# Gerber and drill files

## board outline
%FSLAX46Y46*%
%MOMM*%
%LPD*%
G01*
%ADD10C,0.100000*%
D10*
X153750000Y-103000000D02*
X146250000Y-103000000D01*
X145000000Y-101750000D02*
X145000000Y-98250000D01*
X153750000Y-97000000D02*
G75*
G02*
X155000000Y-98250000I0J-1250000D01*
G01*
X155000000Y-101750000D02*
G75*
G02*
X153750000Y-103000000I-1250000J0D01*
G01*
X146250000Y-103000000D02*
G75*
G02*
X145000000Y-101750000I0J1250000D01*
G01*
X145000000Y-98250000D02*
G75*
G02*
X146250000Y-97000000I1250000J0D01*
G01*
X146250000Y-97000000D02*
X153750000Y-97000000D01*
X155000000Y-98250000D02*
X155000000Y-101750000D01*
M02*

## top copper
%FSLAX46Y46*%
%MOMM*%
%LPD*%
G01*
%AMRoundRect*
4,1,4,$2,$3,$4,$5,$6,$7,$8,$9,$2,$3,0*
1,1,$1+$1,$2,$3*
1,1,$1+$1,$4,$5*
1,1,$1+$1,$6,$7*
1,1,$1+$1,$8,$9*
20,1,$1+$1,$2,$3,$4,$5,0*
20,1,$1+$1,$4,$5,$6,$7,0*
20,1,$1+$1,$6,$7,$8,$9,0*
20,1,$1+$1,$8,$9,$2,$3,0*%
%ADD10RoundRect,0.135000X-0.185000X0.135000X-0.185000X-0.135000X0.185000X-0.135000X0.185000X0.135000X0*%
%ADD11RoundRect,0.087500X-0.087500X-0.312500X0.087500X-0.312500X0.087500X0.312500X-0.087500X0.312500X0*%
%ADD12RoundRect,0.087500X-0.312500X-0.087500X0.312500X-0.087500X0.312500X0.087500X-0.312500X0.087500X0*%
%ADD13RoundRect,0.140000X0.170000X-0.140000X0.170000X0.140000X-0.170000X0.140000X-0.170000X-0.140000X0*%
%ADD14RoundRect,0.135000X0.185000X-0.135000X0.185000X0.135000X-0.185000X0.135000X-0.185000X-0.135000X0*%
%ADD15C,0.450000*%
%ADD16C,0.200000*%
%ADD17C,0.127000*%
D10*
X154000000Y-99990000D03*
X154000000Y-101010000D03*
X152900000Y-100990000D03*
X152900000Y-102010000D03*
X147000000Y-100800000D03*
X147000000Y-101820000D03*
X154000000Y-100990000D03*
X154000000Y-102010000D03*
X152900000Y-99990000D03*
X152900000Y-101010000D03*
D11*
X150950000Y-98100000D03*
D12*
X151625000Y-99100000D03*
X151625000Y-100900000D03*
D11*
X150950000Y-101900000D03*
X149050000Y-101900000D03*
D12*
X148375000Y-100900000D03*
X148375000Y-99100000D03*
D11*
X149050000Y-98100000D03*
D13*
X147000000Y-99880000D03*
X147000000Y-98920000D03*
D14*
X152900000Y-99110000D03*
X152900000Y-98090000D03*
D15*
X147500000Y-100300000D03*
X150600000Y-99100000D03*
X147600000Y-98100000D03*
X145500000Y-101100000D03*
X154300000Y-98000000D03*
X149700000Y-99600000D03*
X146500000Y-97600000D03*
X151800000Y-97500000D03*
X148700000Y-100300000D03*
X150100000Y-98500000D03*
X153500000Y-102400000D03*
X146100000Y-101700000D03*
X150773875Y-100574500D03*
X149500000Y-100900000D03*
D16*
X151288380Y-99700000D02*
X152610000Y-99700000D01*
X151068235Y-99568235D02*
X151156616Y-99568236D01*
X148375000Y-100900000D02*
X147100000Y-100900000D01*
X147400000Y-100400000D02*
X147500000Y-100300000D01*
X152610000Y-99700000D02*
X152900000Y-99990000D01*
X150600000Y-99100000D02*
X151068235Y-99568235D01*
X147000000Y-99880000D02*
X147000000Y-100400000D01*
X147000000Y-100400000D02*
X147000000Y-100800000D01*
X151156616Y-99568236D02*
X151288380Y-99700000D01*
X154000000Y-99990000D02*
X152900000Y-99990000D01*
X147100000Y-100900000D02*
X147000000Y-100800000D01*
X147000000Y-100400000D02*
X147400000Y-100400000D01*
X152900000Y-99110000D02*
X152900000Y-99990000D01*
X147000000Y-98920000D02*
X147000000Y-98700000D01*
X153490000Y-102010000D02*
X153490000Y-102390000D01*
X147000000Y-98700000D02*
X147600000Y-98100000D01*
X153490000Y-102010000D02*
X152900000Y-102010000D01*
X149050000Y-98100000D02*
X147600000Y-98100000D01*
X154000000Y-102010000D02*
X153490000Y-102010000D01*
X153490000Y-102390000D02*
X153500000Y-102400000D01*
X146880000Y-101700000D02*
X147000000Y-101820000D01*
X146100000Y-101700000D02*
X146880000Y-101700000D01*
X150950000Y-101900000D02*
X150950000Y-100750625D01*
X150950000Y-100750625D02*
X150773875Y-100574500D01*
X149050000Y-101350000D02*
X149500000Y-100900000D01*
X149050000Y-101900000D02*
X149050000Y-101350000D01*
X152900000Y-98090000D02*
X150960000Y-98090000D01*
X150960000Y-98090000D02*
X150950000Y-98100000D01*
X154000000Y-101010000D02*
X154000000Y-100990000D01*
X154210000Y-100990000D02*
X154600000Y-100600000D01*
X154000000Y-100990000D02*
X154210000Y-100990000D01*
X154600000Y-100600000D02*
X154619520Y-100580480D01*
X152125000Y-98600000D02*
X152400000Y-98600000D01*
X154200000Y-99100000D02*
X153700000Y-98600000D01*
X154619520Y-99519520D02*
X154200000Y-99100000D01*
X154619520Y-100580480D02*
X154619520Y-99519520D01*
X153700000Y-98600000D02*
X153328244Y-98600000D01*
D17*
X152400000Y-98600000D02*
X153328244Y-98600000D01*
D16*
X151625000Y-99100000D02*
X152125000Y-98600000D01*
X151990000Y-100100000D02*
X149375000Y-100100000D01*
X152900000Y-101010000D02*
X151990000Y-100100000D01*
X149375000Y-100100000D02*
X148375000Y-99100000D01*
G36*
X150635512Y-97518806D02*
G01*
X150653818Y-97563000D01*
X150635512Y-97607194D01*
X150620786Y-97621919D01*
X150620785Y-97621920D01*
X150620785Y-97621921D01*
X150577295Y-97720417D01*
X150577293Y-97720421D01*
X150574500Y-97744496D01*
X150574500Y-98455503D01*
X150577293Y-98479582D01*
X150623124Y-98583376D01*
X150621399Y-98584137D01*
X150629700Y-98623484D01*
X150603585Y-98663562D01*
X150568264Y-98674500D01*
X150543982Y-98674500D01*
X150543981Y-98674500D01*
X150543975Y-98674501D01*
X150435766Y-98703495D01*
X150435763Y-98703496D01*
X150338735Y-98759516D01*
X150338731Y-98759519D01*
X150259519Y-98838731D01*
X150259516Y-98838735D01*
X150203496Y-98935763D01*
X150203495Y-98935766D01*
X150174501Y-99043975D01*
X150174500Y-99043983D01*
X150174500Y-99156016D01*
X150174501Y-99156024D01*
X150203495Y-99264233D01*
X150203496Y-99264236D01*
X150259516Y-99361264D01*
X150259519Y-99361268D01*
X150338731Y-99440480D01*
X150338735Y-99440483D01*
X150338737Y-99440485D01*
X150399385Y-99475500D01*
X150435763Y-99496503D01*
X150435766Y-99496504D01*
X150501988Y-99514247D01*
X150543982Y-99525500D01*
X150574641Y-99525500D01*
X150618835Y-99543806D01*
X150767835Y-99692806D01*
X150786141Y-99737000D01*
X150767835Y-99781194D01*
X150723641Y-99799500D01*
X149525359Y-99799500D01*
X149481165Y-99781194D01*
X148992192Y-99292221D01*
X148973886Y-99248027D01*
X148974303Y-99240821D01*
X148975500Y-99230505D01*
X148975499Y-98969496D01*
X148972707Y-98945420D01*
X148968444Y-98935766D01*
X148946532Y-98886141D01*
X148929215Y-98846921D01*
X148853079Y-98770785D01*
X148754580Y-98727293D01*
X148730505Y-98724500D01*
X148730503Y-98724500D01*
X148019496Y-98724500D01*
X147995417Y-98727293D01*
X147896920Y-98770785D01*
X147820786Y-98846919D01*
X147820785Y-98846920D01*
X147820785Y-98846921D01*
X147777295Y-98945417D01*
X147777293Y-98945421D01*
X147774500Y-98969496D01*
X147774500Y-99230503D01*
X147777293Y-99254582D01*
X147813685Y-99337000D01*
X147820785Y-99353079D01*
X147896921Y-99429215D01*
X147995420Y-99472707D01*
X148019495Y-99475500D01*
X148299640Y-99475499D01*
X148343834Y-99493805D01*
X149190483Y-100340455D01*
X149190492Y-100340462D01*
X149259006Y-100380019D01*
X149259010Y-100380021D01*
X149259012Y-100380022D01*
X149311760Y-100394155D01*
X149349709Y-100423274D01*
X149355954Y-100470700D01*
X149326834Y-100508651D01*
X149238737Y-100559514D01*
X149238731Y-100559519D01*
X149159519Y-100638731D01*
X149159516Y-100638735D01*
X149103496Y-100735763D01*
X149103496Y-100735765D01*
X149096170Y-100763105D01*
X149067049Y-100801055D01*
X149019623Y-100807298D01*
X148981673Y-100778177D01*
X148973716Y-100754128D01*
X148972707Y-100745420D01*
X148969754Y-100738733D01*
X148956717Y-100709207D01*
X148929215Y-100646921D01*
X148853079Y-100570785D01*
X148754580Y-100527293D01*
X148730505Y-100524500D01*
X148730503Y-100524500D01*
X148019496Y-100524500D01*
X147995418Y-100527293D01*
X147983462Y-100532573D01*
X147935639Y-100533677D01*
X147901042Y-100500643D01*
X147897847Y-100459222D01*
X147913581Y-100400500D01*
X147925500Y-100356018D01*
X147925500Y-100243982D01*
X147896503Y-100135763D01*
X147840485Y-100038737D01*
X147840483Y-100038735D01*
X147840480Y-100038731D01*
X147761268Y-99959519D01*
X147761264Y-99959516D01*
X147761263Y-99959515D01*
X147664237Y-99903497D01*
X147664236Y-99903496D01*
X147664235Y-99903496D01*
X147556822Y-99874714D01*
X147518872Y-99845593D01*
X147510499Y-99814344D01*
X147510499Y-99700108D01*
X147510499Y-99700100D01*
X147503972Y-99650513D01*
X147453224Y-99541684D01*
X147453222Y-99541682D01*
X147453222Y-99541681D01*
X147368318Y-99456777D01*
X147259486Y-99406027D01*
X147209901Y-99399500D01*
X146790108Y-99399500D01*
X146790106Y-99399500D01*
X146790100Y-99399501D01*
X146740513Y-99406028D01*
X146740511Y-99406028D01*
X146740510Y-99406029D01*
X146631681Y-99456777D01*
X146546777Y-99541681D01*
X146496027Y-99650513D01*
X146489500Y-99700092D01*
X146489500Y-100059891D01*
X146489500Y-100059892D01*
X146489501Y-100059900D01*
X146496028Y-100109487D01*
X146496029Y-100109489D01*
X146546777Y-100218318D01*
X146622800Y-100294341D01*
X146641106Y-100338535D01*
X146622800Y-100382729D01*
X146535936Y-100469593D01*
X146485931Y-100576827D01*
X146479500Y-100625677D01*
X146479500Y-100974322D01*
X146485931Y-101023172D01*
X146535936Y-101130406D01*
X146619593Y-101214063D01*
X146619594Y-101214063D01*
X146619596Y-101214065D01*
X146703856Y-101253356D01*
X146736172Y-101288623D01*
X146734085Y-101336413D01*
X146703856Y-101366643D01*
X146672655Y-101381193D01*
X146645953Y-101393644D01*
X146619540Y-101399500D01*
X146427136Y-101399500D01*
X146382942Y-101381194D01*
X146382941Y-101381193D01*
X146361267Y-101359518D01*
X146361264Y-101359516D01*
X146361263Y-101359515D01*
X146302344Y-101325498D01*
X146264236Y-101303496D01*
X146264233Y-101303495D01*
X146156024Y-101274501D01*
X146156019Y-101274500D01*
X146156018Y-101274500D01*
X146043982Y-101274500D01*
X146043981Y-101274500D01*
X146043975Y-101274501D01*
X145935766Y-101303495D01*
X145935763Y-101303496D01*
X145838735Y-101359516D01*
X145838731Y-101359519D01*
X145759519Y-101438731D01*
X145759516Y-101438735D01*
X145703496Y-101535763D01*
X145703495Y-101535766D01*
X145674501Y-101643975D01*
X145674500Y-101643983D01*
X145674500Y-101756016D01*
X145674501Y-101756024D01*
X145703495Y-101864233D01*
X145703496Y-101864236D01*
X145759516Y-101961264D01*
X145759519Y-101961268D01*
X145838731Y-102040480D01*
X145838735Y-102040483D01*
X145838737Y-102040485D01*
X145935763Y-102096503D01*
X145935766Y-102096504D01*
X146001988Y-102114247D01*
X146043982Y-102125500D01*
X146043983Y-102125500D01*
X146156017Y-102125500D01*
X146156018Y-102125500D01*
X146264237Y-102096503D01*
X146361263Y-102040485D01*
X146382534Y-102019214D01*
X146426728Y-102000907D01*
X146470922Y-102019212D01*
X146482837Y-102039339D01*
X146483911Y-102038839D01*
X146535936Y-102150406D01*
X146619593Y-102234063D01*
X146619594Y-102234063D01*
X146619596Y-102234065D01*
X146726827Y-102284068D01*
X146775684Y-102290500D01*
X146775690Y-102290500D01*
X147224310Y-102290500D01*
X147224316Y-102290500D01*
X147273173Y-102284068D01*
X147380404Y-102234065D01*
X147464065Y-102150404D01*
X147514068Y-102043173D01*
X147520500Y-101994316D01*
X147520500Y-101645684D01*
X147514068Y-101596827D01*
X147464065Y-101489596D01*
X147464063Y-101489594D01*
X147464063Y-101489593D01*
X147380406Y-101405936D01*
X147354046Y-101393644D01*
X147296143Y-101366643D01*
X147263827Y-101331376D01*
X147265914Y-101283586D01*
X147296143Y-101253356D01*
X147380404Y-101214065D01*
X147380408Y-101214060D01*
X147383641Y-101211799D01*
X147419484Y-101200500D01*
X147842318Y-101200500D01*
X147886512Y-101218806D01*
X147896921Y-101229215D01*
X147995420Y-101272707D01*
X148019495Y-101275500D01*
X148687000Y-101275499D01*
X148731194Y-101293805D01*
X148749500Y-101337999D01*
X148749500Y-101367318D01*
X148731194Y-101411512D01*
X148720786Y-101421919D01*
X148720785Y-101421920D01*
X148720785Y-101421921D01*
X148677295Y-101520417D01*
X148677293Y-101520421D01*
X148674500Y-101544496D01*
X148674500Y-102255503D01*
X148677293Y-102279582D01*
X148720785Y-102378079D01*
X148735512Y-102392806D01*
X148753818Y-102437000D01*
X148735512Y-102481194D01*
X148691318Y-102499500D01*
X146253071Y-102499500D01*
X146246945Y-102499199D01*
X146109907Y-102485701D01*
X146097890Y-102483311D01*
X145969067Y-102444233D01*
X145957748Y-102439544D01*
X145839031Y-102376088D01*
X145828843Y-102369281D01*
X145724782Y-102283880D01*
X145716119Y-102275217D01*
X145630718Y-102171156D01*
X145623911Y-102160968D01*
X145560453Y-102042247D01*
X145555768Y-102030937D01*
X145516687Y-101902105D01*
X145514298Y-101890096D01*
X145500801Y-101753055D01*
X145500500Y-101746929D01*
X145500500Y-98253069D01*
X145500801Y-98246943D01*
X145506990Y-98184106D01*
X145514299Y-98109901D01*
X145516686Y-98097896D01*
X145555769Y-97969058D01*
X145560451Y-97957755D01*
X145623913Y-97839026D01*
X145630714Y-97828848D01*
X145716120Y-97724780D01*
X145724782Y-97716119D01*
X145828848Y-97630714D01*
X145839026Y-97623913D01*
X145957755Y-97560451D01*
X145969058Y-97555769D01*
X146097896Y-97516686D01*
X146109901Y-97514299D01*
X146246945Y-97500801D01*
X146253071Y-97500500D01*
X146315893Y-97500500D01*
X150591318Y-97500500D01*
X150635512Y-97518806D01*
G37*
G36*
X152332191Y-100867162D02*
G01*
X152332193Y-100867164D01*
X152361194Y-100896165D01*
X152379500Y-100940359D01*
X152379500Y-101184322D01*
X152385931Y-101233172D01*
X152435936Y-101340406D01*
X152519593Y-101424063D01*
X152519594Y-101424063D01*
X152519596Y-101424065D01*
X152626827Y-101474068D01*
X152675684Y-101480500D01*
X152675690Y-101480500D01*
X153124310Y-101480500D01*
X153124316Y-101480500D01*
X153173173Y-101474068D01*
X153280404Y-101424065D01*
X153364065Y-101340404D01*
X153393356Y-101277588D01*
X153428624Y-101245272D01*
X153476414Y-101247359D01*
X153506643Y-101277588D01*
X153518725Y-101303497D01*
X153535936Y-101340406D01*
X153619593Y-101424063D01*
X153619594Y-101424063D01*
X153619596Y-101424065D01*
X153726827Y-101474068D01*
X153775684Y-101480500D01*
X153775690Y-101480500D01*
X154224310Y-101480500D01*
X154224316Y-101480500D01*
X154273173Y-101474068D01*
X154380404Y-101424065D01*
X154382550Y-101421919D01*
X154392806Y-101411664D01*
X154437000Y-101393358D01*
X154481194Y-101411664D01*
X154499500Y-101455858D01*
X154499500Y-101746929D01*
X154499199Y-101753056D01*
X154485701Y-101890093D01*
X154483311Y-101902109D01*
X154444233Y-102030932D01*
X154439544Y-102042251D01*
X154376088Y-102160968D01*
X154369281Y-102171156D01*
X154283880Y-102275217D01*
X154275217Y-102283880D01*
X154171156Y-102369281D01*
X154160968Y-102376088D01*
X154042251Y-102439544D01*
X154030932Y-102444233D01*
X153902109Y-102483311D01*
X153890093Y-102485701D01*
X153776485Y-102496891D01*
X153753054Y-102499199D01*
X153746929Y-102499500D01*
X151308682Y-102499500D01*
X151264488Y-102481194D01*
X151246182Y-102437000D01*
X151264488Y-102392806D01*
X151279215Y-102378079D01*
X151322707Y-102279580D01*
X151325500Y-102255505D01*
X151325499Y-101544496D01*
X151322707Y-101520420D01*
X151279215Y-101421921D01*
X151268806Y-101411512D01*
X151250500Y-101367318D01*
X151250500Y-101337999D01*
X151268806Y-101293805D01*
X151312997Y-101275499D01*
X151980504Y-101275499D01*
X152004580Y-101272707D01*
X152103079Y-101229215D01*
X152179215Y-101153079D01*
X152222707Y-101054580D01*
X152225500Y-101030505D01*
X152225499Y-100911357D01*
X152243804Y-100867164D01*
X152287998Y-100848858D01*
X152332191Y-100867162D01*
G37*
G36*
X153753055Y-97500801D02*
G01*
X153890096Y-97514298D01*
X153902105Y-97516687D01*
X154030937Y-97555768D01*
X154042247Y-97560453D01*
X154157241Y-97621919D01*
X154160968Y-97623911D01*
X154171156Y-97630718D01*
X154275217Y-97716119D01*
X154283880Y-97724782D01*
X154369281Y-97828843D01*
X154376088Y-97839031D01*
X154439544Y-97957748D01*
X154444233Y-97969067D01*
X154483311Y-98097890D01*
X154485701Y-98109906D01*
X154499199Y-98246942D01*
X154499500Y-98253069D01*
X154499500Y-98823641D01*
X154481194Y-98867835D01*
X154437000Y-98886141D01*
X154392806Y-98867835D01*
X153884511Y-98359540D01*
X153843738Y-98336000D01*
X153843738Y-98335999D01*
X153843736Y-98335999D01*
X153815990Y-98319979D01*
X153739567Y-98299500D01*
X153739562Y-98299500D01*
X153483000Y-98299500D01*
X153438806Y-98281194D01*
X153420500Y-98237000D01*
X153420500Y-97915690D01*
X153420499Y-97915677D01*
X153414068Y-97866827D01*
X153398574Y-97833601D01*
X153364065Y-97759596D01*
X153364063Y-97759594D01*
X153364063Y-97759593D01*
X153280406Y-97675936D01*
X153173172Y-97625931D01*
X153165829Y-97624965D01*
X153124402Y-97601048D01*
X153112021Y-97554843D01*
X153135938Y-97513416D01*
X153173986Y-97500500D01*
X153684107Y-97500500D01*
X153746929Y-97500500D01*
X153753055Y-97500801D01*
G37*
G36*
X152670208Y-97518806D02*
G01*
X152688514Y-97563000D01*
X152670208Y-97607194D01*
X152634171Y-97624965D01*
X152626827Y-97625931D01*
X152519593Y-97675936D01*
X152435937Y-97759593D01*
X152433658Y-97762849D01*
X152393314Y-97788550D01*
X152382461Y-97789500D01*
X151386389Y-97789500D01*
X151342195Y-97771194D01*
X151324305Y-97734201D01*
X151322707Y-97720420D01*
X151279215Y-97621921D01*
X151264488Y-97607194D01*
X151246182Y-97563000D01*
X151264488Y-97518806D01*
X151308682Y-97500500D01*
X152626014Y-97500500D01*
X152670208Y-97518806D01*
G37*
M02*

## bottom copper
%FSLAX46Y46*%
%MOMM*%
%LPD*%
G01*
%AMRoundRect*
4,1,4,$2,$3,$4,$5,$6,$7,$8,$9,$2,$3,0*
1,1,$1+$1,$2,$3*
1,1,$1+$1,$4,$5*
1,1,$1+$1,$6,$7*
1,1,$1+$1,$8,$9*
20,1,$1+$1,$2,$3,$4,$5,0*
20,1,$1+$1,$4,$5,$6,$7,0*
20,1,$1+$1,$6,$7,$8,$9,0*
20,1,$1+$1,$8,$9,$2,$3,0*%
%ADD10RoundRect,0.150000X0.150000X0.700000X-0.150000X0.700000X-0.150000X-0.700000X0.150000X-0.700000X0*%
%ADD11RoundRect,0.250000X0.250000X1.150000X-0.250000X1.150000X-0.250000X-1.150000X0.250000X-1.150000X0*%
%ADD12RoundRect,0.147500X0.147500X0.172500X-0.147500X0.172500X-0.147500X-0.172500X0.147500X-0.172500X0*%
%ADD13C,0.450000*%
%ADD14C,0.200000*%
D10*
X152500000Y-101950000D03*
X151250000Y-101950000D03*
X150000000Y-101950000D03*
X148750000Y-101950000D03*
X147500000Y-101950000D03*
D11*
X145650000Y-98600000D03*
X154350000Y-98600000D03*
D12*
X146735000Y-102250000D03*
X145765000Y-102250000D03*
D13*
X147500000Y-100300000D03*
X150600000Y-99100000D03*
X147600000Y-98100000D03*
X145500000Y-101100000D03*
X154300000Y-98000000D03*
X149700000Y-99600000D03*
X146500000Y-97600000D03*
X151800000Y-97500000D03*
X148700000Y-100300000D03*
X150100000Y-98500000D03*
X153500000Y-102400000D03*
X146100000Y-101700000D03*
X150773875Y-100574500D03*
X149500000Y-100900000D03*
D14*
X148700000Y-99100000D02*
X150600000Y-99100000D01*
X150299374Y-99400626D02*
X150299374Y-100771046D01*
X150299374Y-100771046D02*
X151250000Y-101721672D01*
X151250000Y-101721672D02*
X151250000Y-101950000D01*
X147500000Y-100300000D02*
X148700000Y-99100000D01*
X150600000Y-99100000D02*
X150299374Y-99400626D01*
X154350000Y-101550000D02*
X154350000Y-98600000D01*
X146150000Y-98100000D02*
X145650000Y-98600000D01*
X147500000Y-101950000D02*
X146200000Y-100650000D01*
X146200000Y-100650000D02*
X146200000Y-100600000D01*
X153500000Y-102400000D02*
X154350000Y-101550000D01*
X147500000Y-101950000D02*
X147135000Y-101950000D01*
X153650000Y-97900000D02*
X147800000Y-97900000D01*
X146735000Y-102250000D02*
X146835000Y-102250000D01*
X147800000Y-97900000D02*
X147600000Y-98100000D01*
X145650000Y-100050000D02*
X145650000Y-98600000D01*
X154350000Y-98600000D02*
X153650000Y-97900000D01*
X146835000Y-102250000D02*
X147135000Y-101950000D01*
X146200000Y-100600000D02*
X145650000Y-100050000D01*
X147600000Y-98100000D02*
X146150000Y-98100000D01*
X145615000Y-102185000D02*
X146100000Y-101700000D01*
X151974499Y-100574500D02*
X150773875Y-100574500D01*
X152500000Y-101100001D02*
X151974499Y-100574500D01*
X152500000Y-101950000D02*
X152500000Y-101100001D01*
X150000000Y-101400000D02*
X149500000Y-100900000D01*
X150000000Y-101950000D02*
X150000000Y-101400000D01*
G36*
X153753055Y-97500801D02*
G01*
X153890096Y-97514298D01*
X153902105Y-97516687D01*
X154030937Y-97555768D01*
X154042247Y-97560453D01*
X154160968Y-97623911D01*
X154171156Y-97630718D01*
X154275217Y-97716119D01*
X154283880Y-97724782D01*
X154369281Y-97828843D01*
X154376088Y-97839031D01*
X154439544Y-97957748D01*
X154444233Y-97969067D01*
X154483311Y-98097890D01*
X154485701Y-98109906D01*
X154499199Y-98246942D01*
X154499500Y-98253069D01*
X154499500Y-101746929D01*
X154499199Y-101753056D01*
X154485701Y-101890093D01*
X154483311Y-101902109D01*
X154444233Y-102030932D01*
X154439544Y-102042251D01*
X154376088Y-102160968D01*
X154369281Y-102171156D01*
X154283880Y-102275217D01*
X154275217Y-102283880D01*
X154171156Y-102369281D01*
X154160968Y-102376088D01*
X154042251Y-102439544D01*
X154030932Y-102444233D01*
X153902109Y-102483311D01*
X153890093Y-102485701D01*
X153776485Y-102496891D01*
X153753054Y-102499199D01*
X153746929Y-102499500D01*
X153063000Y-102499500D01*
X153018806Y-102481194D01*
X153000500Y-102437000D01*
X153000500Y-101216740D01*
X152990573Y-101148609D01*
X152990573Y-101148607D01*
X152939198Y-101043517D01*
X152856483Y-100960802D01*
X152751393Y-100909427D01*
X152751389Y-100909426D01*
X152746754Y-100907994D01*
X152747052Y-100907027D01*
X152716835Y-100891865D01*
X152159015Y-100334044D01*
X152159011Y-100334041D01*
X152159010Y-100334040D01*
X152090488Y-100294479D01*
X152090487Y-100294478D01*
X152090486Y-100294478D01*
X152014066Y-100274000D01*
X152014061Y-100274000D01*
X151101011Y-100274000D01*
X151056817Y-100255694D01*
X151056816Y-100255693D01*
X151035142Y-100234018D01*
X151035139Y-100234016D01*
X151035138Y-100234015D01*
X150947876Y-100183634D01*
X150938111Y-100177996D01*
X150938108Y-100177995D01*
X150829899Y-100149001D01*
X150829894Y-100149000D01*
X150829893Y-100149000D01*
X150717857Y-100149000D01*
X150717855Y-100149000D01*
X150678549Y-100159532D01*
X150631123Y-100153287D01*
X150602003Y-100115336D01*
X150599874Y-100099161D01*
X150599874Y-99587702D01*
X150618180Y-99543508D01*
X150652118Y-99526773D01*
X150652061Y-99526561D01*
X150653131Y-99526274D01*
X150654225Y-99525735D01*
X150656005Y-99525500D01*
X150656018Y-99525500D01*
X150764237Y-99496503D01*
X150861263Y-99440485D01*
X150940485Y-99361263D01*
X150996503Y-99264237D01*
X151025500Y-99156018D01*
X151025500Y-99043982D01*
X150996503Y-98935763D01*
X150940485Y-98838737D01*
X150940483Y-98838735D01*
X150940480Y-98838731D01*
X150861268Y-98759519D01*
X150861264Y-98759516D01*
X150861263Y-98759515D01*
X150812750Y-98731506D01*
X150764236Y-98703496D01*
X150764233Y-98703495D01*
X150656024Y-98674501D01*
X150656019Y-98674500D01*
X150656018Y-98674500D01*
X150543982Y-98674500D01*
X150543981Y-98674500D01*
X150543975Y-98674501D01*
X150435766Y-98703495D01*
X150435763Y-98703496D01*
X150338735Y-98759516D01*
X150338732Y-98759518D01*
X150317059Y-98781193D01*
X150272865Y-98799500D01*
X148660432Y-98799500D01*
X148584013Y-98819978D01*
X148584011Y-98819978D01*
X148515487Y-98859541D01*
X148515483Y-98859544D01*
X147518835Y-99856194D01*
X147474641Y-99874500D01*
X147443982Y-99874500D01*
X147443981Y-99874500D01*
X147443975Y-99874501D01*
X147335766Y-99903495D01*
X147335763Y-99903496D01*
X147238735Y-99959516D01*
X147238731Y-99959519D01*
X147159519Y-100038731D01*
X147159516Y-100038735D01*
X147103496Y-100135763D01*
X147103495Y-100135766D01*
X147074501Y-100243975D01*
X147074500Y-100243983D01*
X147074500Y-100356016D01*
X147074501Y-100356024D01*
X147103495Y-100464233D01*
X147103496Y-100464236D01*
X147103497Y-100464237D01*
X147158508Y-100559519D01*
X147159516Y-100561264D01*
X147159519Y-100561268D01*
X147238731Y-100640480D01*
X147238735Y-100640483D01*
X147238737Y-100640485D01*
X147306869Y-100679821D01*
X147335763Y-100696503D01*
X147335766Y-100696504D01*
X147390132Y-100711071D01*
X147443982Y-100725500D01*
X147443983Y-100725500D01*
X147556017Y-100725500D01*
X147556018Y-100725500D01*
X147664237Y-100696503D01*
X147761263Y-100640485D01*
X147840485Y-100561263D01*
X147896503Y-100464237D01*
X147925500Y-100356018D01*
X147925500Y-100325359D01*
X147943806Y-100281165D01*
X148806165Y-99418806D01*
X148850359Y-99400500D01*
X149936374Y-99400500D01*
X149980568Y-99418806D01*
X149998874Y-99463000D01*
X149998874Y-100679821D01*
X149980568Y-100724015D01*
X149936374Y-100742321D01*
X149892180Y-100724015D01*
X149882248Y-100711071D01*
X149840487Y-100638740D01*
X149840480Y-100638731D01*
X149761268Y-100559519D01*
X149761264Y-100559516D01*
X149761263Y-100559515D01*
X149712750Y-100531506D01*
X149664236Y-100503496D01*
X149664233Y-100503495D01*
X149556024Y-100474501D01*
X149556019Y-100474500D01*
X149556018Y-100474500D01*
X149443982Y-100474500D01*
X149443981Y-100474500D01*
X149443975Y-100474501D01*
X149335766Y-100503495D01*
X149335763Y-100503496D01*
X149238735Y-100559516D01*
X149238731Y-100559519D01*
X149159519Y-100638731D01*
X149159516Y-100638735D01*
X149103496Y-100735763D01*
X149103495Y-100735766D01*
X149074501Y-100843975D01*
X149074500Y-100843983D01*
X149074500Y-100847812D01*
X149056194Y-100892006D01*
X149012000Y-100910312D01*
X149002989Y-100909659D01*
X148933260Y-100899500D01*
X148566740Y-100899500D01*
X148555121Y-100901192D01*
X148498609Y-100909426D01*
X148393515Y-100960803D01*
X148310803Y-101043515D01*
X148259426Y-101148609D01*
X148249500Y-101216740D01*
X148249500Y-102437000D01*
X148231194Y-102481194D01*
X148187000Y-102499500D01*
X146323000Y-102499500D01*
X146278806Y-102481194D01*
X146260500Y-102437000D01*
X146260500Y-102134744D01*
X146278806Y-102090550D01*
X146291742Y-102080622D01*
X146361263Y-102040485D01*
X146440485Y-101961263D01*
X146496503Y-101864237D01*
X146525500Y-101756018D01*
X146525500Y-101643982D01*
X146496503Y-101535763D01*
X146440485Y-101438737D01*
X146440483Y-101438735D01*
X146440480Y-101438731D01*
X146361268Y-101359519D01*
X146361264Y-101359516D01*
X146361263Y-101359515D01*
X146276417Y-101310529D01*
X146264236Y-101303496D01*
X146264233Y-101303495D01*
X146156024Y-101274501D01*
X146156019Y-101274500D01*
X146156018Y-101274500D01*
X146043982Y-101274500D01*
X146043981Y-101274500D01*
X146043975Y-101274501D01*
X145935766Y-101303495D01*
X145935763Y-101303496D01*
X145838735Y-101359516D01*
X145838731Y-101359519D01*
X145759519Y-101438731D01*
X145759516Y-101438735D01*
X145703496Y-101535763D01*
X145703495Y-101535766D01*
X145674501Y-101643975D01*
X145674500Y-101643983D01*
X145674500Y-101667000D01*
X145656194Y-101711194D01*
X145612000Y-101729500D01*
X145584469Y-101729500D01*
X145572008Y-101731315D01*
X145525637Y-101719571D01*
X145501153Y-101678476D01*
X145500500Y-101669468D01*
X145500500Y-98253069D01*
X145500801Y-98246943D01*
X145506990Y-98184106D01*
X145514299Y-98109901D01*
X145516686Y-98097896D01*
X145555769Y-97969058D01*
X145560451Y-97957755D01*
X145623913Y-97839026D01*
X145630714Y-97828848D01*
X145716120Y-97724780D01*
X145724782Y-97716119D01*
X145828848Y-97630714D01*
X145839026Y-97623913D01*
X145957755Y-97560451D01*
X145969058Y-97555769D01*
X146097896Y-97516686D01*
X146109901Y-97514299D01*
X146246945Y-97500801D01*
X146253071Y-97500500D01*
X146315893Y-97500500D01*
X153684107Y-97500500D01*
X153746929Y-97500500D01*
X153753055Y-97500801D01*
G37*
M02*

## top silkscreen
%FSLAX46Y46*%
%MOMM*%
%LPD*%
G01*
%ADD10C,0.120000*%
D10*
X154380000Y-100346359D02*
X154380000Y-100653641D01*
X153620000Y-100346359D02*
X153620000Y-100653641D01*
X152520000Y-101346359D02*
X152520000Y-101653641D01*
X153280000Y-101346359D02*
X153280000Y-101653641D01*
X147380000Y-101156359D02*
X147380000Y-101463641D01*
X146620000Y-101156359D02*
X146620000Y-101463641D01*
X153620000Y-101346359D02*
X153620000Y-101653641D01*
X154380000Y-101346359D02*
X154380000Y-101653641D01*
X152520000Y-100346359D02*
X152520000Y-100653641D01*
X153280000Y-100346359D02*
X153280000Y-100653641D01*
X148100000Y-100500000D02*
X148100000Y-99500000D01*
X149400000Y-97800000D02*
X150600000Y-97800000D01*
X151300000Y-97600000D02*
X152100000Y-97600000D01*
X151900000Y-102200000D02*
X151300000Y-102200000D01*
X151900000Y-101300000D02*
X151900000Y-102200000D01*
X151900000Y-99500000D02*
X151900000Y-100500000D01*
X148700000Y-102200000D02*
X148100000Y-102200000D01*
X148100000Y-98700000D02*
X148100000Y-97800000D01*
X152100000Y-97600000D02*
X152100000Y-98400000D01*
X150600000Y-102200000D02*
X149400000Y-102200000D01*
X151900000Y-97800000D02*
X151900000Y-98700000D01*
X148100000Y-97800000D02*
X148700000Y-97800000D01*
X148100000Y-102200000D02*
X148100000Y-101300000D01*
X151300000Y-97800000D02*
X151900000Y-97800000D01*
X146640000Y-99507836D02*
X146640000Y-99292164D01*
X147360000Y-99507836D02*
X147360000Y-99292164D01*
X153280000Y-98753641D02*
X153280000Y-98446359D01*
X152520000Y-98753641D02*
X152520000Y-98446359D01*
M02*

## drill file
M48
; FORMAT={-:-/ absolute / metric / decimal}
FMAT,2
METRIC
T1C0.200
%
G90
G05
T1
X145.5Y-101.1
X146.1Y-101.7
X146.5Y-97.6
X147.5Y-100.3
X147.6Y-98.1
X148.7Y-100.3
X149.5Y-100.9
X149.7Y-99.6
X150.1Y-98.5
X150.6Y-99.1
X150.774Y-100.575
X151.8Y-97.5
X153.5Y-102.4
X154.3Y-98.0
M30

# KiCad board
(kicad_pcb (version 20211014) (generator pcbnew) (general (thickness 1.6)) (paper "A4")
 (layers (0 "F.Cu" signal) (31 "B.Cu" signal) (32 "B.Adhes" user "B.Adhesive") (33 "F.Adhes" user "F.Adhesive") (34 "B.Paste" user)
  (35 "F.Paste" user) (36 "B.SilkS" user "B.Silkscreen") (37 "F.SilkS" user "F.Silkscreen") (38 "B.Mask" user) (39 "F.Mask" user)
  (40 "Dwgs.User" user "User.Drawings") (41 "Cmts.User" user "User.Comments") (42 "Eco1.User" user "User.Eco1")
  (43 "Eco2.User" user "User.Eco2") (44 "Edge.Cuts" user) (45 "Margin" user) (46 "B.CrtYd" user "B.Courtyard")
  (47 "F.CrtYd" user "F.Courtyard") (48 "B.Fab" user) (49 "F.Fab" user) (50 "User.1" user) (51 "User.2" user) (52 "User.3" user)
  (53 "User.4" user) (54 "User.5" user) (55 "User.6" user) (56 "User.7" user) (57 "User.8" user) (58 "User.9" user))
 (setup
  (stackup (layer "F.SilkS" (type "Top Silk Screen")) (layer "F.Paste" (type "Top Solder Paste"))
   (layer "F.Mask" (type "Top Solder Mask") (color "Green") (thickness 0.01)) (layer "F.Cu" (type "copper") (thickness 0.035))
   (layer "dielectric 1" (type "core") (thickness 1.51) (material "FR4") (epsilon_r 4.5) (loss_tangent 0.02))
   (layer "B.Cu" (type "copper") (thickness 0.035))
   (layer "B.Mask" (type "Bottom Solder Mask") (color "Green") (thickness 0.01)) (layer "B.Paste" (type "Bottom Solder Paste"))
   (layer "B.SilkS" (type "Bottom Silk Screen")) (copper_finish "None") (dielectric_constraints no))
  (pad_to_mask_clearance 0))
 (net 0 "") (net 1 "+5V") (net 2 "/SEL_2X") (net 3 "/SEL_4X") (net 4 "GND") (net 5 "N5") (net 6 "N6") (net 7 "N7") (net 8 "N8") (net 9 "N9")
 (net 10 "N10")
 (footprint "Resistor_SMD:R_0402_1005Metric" (layer "F.Cu") (at 154 100.5 -90)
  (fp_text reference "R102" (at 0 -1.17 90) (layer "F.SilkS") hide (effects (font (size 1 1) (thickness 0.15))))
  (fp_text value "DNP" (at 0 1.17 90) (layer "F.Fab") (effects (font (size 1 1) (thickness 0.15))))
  (fp_line (start -0.153641 -0.38) (end 0.153641 -0.38) (layer "F.SilkS") (width 0.12))
  (fp_line (start -0.153641 0.38) (end 0.153641 0.38) (layer "F.SilkS") (width 0.12))
  (pad "1" smd roundrect locked (at -0.51 0 270) (size 0.54 0.64) (layers "F.Cu" "F.Paste" "F.Mask") (roundrect_rratio 0.25) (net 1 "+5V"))
  (pad "2" smd roundrect locked (at 0.51 0 270) (size 0.54 0.64) (layers "F.Cu" "F.Paste" "F.Mask") (roundrect_rratio 0.25)
   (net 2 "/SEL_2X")))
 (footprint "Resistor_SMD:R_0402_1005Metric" (layer "F.Cu") (at 152.9 101.5 -90)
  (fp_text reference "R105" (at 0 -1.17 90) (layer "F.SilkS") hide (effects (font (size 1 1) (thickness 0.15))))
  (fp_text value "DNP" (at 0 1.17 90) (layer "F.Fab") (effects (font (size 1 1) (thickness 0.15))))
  (fp_line (start -0.153641 0.38) (end 0.153641 0.38) (layer "F.SilkS") (width 0.12))
  (fp_line (start -0.153641 -0.38) (end 0.153641 -0.38) (layer "F.SilkS") (width 0.12))
  (pad "1" smd roundrect locked (at -0.51 0 270) (size 0.54 0.64) (layers "F.Cu" "F.Paste" "F.Mask") (roundrect_rratio 0.25)
   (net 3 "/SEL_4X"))
  (pad "2" smd roundrect locked (at 0.51 0 270) (size 0.54 0.64) (layers "F.Cu" "F.Paste" "F.Mask") (roundrect_rratio 0.25) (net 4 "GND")))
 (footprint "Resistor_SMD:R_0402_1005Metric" (layer "F.Cu") (at 147 101.31 -90)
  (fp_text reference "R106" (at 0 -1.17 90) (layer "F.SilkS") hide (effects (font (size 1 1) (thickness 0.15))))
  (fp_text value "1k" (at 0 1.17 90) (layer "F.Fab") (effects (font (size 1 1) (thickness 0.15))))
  (fp_line (start -0.153641 -0.38) (end 0.153641 -0.38) (layer "F.SilkS") (width 0.12))
  (fp_line (start -0.153641 0.38) (end 0.153641 0.38) (layer "F.SilkS") (width 0.12))
  (pad "1" smd roundrect locked (at -0.51 0 270) (size 0.54 0.64) (layers "F.Cu" "F.Paste" "F.Mask") (roundrect_rratio 0.25) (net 1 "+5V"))
  (pad "2" smd roundrect locked (at 0.51 0 270) (size 0.54 0.64) (layers "F.Cu" "F.Paste" "F.Mask") (roundrect_rratio 0.25) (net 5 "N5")))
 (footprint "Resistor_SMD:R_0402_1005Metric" (layer "F.Cu") (at 154 101.5 -90)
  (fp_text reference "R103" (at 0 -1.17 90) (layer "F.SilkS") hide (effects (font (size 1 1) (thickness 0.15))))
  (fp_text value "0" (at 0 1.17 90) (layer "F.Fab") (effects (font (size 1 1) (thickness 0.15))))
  (fp_line (start -0.153641 0.38) (end 0.153641 0.38) (layer "F.SilkS") (width 0.12))
  (fp_line (start -0.153641 -0.38) (end 0.153641 -0.38) (layer "F.SilkS") (width 0.12))
  (pad "1" smd roundrect locked (at -0.51 0 270) (size 0.54 0.64) (layers "F.Cu" "F.Paste" "F.Mask") (roundrect_rratio 0.25)
   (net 2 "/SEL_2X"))
  (pad "2" smd roundrect locked (at 0.51 0 270) (size 0.54 0.64) (layers "F.Cu" "F.Paste" "F.Mask") (roundrect_rratio 0.25) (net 4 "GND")))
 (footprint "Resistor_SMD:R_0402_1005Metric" (layer "F.Cu") (at 152.9 100.5 -90)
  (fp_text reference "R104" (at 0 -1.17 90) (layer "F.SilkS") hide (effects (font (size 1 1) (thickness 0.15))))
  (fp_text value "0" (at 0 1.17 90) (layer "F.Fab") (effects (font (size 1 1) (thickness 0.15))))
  (fp_line (start -0.153641 0.38) (end 0.153641 0.38) (layer "F.SilkS") (width 0.12))
  (fp_line (start -0.153641 -0.38) (end 0.153641 -0.38) (layer "F.SilkS") (width 0.12))
  (pad "1" smd roundrect locked (at -0.51 0 270) (size 0.54 0.64) (layers "F.Cu" "F.Paste" "F.Mask") (roundrect_rratio 0.25) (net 1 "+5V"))
  (pad "2" smd roundrect locked (at 0.51 0 270) (size 0.54 0.64) (layers "F.Cu" "F.Paste" "F.Mask") (roundrect_rratio 0.25)
   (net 3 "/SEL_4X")))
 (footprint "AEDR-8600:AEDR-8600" (layer "F.Cu") (at 150 100)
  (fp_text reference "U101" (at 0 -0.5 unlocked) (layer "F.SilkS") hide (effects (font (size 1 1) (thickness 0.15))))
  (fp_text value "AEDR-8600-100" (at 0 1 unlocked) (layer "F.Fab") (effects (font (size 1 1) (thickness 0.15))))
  (fp_line (start -1.9 0.5) (end -1.9 -0.5) (layer "F.SilkS") (width 0.12))
  (fp_line (start -0.6 -2.2) (end 0.6 -2.2) (layer "F.SilkS") (width 0.12))
  (fp_line (start 1.3 -2.4) (end 2.1 -2.4) (layer "F.SilkS") (width 0.12))
  (fp_line (start 1.9 2.2) (end 1.3 2.2) (layer "F.SilkS") (width 0.12))
  (fp_line (start 1.9 1.3) (end 1.9 2.2) (layer "F.SilkS") (width 0.12))
  (fp_line (start 1.9 -0.5) (end 1.9 0.5) (layer "F.SilkS") (width 0.12))
  (fp_line (start -1.3 2.2) (end -1.9 2.2) (layer "F.SilkS") (width 0.12))
  (fp_line (start -1.9 -1.3) (end -1.9 -2.2) (layer "F.SilkS") (width 0.12))
  (fp_line (start 2.1 -2.4) (end 2.1 -1.6) (layer "F.SilkS") (width 0.12))
  (fp_line (start 0.6 2.2) (end -0.6 2.2) (layer "F.SilkS") (width 0.12))
  (fp_line (start 1.9 -2.2) (end 1.9 -1.3) (layer "F.SilkS") (width 0.12))
  (fp_line (start -1.9 -2.2) (end -1.3 -2.2) (layer "F.SilkS") (width 0.12))
  (fp_line (start -1.9 2.2) (end -1.9 1.3) (layer "F.SilkS") (width 0.12))
  (fp_line (start 1.3 -2.2) (end 1.9 -2.2) (layer "F.SilkS") (width 0.12))
  (pad "1" smd roundrect (at 0.95 -1.9) (size 0.35 0.8) (layers "F.Cu" "F.Paste" "F.Mask") (roundrect_rratio 0.25) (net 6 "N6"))
  (pad "2" smd roundrect (at 1.625 -0.9) (size 0.8 0.35) (layers "F.Cu" "F.Paste" "F.Mask") (roundrect_rratio 0.25) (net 2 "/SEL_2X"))
  (pad "3" smd roundrect (at 1.625 0.9) (size 0.8 0.35) (layers "F.Cu" "F.Paste" "F.Mask") (roundrect_rratio 0.25) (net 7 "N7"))
  (pad "4" smd roundrect (at 0.95 1.9) (size 0.35 0.8) (layers "F.Cu" "F.Paste" "F.Mask") (roundrect_rratio 0.25) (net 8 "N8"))
  (pad "5" smd roundrect (at -0.95 1.9) (size 0.35 0.8) (layers "F.Cu" "F.Paste" "F.Mask") (roundrect_rratio 0.25) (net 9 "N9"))
  (pad "6" smd roundrect (at -1.625 0.9) (size 0.8 0.35) (layers "F.Cu" "F.Paste" "F.Mask") (roundrect_rratio 0.25) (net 1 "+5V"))
  (pad "7" smd roundrect (at -1.625 -0.9) (size 0.8 0.35) (layers "F.Cu" "F.Paste" "F.Mask") (roundrect_rratio 0.25) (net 3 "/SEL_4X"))
  (pad "8" smd roundrect (at -0.95 -1.9) (size 0.35 0.8) (layers "F.Cu" "F.Paste" "F.Mask") (roundrect_rratio 0.25) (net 4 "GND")))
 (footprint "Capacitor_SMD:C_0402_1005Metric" (layer "F.Cu") (at 147 99.4 90)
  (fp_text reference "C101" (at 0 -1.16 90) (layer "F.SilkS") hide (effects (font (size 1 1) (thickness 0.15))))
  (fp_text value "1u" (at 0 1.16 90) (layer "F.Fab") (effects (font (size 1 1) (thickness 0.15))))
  (fp_line (start -0.107836 -0.36) (end 0.107836 -0.36) (layer "F.SilkS") (width 0.12))
  (fp_line (start -0.107836 0.36) (end 0.107836 0.36) (layer "F.SilkS") (width 0.12))
  (pad "1" smd roundrect locked (at -0.48 0 90) (size 0.56 0.62) (layers "F.Cu" "F.Paste" "F.Mask") (roundrect_rratio 0.25) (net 1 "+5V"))
  (pad "2" smd roundrect locked (at 0.48 0 90) (size 0.56 0.62) (layers "F.Cu" "F.Paste" "F.Mask") (roundrect_rratio 0.25) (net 4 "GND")))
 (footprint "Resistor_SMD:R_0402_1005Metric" (layer "F.Cu") (at 152.9 98.6 90)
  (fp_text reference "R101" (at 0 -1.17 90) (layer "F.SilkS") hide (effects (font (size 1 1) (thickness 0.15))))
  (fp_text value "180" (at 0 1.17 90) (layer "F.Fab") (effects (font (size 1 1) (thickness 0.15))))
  (fp_line (start -0.153641 0.38) (end 0.153641 0.38) (layer "F.SilkS") (width 0.12))
  (fp_line (start -0.153641 -0.38) (end 0.153641 -0.38) (layer "F.SilkS") (width 0.12))
  (pad "1" smd roundrect locked (at -0.51 0 90) (size 0.54 0.64) (layers "F.Cu" "F.Paste" "F.Mask") (roundrect_rratio 0.25) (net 1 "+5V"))
  (pad "2" smd roundrect locked (at 0.51 0 90) (size 0.54 0.64) (layers "F.Cu" "F.Paste" "F.Mask") (roundrect_rratio 0.25) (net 6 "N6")))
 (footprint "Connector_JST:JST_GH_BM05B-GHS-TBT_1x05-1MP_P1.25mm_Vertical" (layer "B.Cu") (at 150 100 180)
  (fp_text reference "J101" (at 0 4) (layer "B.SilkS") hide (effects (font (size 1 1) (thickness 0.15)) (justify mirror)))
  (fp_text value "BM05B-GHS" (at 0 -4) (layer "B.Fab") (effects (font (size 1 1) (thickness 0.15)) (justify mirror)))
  (pad "1" smd roundrect locked (at -2.5 -1.95 180) (size 0.6 1.7) (layers "B.Cu" "B.Paste" "B.Mask") (roundrect_rratio 0.25) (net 8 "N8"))
  (pad "2" smd roundrect locked (at -1.25 -1.95 180) (size 0.6 1.7) (layers "B.Cu" "B.Paste" "B.Mask") (roundrect_rratio 0.25) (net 1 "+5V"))
  (pad "3" smd roundrect locked (at 0 -1.95 180) (size 0.6 1.7) (layers "B.Cu" "B.Paste" "B.Mask") (roundrect_rratio 0.25) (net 9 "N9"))
  (pad "4" smd roundrect locked (at 1.25 -1.95 180) (size 0.6 1.7) (layers "B.Cu" "B.Paste" "B.Mask") (roundrect_rratio 0.25) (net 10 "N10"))
  (pad "5" smd roundrect locked (at 2.5 -1.95 180) (size 0.6 1.7) (layers "B.Cu" "B.Paste" "B.Mask") (roundrect_rratio 0.25) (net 4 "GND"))
  (pad "MP" smd roundrect locked (at 4.35 1.4 180) (size 1 2.8) (layers "B.Cu" "B.Paste" "B.Mask") (roundrect_rratio 0.25) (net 4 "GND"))
  (pad "MP" smd roundrect locked (at -4.35 1.4 180) (size 1 2.8) (layers "B.Cu" "B.Paste" "B.Mask") (roundrect_rratio 0.25) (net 4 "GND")))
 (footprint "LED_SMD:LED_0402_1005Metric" (layer "B.Cu") (at 146.25 102.25 180)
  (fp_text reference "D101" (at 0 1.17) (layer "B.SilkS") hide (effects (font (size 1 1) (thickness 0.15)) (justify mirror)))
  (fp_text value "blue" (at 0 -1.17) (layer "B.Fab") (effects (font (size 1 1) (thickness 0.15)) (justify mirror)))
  (pad "1" smd roundrect locked (at -0.485 0 180) (size 0.59 0.64) (layers "B.Cu" "B.Paste" "B.Mask") (roundrect_rratio 0.25) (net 4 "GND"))
  (pad "2" smd roundrect locked (at 0.485 0 180) (size 0.59 0.64) (layers "B.Cu" "B.Paste" "B.Mask") (roundrect_rratio 0.25) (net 5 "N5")))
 (gr_line (start 153.75 103) (end 146.25 103) (layer "Edge.Cuts") (width 0.1))
 (gr_line (start 145 101.75) (end 145 98.25) (layer "Edge.Cuts") (width 0.1))
 (gr_arc (start 153.75 97) (mid 154.633883 97.366117) (end 155 98.25) (layer "Edge.Cuts") (width 0.1))
 (gr_arc (start 155 101.75) (mid 154.633883 102.633883) (end 153.75 103) (layer "Edge.Cuts") (width 0.1))
 (gr_arc (start 146.25 103) (mid 145.366117 102.633883) (end 145 101.75) (layer "Edge.Cuts") (width 0.1))
 (gr_arc (start 145 98.25) (mid 145.366117 97.366117) (end 146.25 97) (layer "Edge.Cuts") (width 0.1))
 (gr_line (start 146.25 97) (end 153.75 97) (layer "Edge.Cuts") (width 0.1))
 (gr_line (start 155 98.25) (end 155 101.75) (layer "Edge.Cuts") (width 0.1))
 (segment (start 151.28838 99.7) (end 152.61 99.7) (width 0.2) (layer "F.Cu") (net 1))
 (segment (start 151.068235 99.568235) (end 151.156616 99.568236) (width 0.2) (layer "F.Cu") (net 1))
 (segment (start 148.375 100.9) (end 147.1 100.9) (width 0.2) (layer "F.Cu") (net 1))
 (segment (start 147.4 100.4) (end 147.5 100.3) (width 0.2) (layer "F.Cu") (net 1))
 (segment (start 152.61 99.7) (end 152.9 99.99) (width 0.2) (layer "F.Cu") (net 1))
 (segment (start 150.6 99.1) (end 151.068235 99.568235) (width 0.2) (layer "F.Cu") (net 1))
 (segment (start 147 99.88) (end 147 100.4) (width 0.2) (layer "F.Cu") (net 1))
 (segment (start 147 100.4) (end 147 100.8) (width 0.2) (layer "F.Cu") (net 1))
 (segment (start 151.156616 99.568236) (end 151.28838 99.7) (width 0.2) (layer "F.Cu") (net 1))
 (segment (start 154 99.99) (end 152.9 99.99) (width 0.2) (layer "F.Cu") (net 1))
 (segment (start 147.1 100.9) (end 147 100.8) (width 0.2) (layer "F.Cu") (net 1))
 (segment (start 147 100.4) (end 147.4 100.4) (width 0.2) (layer "F.Cu") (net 1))
 (segment (start 152.9 99.11) (end 152.9 99.99) (width 0.2) (layer "F.Cu") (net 1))
 (via (at 147.5 100.3) (size 0.45) (drill 0.2) (layers "F.Cu" "B.Cu") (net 1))
 (via (at 150.6 99.1) (size 0.45) (drill 0.2) (layers "F.Cu" "B.Cu") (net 1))
 (segment (start 148.7 99.1) (end 150.6 99.1) (width 0.2) (layer "B.Cu") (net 1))
 (segment (start 150.299374 99.400626) (end 150.299374 100.771046) (width 0.2) (layer "B.Cu") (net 1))
 (segment (start 150.299374 100.771046) (end 151.25 101.721672) (width 0.2) (layer "B.Cu") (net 1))
 (segment (start 151.25 101.721672) (end 151.25 101.95) (width 0.2) (layer "B.Cu") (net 1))
 (segment (start 147.5 100.3) (end 148.7 99.1) (width 0.2) (layer "B.Cu") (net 1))
 (segment (start 150.6 99.1) (end 150.299374 99.400626) (width 0.2) (layer "B.Cu") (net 1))
 (segment (start 147 98.92) (end 147 98.7) (width 0.2) (layer "F.Cu") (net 4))
 (segment (start 153.49 102.01) (end 153.49 102.39) (width 0.2) (layer "F.Cu") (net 4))
 (segment (start 147 98.7) (end 147.6 98.1) (width 0.2) (layer "F.Cu") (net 4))
 (segment (start 153.49 102.01) (end 152.9 102.01) (width 0.2) (layer "F.Cu") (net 4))
 (segment (start 149.05 98.1) (end 147.6 98.1) (width 0.2) (layer "F.Cu") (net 4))
 (segment (start 154 102.01) (end 153.49 102.01) (width 0.2) (layer "F.Cu") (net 4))
 (segment (start 153.49 102.39) (end 153.5 102.4) (width 0.2) (layer "F.Cu") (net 4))
 (via (at 147.6 98.1) (size 0.45) (drill 0.2) (layers "F.Cu" "B.Cu") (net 4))
 (via (at 145.5 101.1) (size 0.45) (drill 0.2) (layers "F.Cu" "B.Cu") (free) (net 4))
 (via (at 154.3 98) (size 0.45) (drill 0.2) (layers "F.Cu" "B.Cu") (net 4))
 (via (at 149.7 99.6) (size 0.45) (drill 0.2) (layers "F.Cu" "B.Cu") (free) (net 4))
 (via (at 146.5 97.6) (size 0.45) (drill 0.2) (layers "F.Cu" "B.Cu") (free) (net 4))
 (via (at 151.8 97.5) (size 0.45) (drill 0.2) (layers "F.Cu" "B.Cu") (free) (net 4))
 (via (at 148.7 100.3) (size 0.45) (drill 0.2) (layers "F.Cu" "B.Cu") (free) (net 4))
 (via (at 150.1 98.5) (size 0.45) (drill 0.2) (layers "F.Cu" "B.Cu") (free) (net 4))
 (via (at 153.5 102.4) (size 0.45) (drill 0.2) (layers "F.Cu" "B.Cu") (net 4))
 (segment (start 154.35 101.55) (end 154.35 98.6) (width 0.2) (layer "B.Cu") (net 4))
 (segment (start 146.15 98.1) (end 145.65 98.6) (width 0.2) (layer "B.Cu") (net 4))
 (segment (start 147.5 101.95) (end 146.2 100.65) (width 0.2) (layer "B.Cu") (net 4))
 (segment (start 146.2 100.65) (end 146.2 100.6) (width 0.2) (layer "B.Cu") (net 4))
 (segment (start 153.5 102.4) (end 154.35 101.55) (width 0.2) (layer "B.Cu") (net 4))
 (segment (start 147.5 101.95) (end 147.135 101.95) (width 0.2) (layer "B.Cu") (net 4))
 (segment (start 153.65 97.9) (end 147.8 97.9) (width 0.2) (layer "B.Cu") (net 4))
 (segment (start 146.735 102.25) (end 146.835 102.25) (width 0.2) (layer "B.Cu") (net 4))
 (segment (start 147.8 97.9) (end 147.6 98.1) (width 0.2) (layer "B.Cu") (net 4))
 (segment (start 145.65 100.05) (end 145.65 98.6) (width 0.2) (layer "B.Cu") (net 4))
 (segment (start 154.35 98.6) (end 153.65 97.9) (width 0.2) (layer "B.Cu") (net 4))
 (segment (start 146.835 102.25) (end 147.135 101.95) (width 0.2) (layer "B.Cu") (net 4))
 (segment (start 146.2 100.6) (end 145.65 100.05) (width 0.2) (layer "B.Cu") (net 4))
 (segment (start 147.6 98.1) (end 146.15 98.1) (width 0.2) (layer "B.Cu") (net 4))
 (segment (start 146.88 101.7) (end 147 101.82) (width 0.2) (layer "F.Cu") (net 5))
 (segment (start 146.1 101.7) (end 146.88 101.7) (width 0.2) (layer "F.Cu") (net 5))
 (via (at 146.1 101.7) (size 0.45) (drill 0.2) (layers "F.Cu" "B.Cu") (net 5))
 (segment (start 145.615 102.185) (end 146.1 101.7) (width 0.2) (layer "B.Cu") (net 5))
 (segment (start 150.95 101.9) (end 150.95 100.750625) (width 0.2) (layer "F.Cu") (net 8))
 (segment (start 150.95 100.750625) (end 150.773875 100.5745) (width 0.2) (layer "F.Cu") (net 8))
 (via (at 150.773875 100.5745) (size 0.45) (drill 0.2) (layers "F.Cu" "B.Cu") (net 8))
 (segment (start 151.974499 100.5745) (end 150.773875 100.5745) (width 0.2) (layer "B.Cu") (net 8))
 (segment (start 152.5 101.100001) (end 151.974499 100.5745) (width 0.2) (layer "B.Cu") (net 8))
 (segment (start 152.5 101.95) (end 152.5 101.100001) (width 0.2) (layer "B.Cu") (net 8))
 (segment (start 149.05 101.35) (end 149.5 100.9) (width 0.2) (layer "F.Cu") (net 9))
 (segment (start 149.05 101.9) (end 149.05 101.35) (width 0.2) (layer "F.Cu") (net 9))
 (via (at 149.5 100.9) (size 0.45) (drill 0.2) (layers "F.Cu" "B.Cu") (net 9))
 (segment (start 150 101.4) (end 149.5 100.9) (width 0.2) (layer "B.Cu") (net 9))
 (segment (start 150 101.95) (end 150 101.4) (width 0.2) (layer "B.Cu") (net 9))
 (segment (start 152.9 98.09) (end 150.96 98.09) (width 0.2) (layer "F.Cu") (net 6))
 (segment (start 150.96 98.09) (end 150.95 98.1) (width 0.2) (layer "F.Cu") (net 6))
 (segment (start 154 101.01) (end 154 100.99) (width 0.2) (layer "F.Cu") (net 2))
 (segment (start 154.21 100.99) (end 154.6 100.6) (width 0.2) (layer "F.Cu") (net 2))
 (segment (start 154 100.99) (end 154.21 100.99) (width 0.2) (layer "F.Cu") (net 2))
 (segment (start 154.6 100.6) (end 154.61952 100.58048) (width 0.2) (layer "F.Cu") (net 2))
 (segment (start 152.125 98.6) (end 152.4 98.6) (width 0.2) (layer "F.Cu") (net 2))
 (segment (start 154.2 99.1) (end 153.7 98.6) (width 0.2) (layer "F.Cu") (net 2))
 (segment (start 154.61952 99.51952) (end 154.2 99.1) (width 0.2) (layer "F.Cu") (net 2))
 (segment (start 154.61952 100.58048) (end 154.61952 99.51952) (width 0.2) (layer "F.Cu") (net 2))
 (segment (start 153.7 98.6) (end 153.328244 98.6) (width 0.2) (layer "F.Cu") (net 2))
 (segment (start 152.4 98.6) (end 153.328244 98.6) (width 0.127) (layer "F.Cu") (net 2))
 (segment (start 151.625 99.1) (end 152.125 98.6) (width 0.2) (layer "F.Cu") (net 2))
 (segment (start 151.99 100.1) (end 149.375 100.1) (width 0.2) (layer "F.Cu") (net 3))
 (segment (start 152.9 101.01) (end 151.99 100.1) (width 0.2) (layer "F.Cu") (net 3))
 (segment (start 149.375 100.1) (end 148.375 99.1) (width 0.2) (layer "F.Cu") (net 3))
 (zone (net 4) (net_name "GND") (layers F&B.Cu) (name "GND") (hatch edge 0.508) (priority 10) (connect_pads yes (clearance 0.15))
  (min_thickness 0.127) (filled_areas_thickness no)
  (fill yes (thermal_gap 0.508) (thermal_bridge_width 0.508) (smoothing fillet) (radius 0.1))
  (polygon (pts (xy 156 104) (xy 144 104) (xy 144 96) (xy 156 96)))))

